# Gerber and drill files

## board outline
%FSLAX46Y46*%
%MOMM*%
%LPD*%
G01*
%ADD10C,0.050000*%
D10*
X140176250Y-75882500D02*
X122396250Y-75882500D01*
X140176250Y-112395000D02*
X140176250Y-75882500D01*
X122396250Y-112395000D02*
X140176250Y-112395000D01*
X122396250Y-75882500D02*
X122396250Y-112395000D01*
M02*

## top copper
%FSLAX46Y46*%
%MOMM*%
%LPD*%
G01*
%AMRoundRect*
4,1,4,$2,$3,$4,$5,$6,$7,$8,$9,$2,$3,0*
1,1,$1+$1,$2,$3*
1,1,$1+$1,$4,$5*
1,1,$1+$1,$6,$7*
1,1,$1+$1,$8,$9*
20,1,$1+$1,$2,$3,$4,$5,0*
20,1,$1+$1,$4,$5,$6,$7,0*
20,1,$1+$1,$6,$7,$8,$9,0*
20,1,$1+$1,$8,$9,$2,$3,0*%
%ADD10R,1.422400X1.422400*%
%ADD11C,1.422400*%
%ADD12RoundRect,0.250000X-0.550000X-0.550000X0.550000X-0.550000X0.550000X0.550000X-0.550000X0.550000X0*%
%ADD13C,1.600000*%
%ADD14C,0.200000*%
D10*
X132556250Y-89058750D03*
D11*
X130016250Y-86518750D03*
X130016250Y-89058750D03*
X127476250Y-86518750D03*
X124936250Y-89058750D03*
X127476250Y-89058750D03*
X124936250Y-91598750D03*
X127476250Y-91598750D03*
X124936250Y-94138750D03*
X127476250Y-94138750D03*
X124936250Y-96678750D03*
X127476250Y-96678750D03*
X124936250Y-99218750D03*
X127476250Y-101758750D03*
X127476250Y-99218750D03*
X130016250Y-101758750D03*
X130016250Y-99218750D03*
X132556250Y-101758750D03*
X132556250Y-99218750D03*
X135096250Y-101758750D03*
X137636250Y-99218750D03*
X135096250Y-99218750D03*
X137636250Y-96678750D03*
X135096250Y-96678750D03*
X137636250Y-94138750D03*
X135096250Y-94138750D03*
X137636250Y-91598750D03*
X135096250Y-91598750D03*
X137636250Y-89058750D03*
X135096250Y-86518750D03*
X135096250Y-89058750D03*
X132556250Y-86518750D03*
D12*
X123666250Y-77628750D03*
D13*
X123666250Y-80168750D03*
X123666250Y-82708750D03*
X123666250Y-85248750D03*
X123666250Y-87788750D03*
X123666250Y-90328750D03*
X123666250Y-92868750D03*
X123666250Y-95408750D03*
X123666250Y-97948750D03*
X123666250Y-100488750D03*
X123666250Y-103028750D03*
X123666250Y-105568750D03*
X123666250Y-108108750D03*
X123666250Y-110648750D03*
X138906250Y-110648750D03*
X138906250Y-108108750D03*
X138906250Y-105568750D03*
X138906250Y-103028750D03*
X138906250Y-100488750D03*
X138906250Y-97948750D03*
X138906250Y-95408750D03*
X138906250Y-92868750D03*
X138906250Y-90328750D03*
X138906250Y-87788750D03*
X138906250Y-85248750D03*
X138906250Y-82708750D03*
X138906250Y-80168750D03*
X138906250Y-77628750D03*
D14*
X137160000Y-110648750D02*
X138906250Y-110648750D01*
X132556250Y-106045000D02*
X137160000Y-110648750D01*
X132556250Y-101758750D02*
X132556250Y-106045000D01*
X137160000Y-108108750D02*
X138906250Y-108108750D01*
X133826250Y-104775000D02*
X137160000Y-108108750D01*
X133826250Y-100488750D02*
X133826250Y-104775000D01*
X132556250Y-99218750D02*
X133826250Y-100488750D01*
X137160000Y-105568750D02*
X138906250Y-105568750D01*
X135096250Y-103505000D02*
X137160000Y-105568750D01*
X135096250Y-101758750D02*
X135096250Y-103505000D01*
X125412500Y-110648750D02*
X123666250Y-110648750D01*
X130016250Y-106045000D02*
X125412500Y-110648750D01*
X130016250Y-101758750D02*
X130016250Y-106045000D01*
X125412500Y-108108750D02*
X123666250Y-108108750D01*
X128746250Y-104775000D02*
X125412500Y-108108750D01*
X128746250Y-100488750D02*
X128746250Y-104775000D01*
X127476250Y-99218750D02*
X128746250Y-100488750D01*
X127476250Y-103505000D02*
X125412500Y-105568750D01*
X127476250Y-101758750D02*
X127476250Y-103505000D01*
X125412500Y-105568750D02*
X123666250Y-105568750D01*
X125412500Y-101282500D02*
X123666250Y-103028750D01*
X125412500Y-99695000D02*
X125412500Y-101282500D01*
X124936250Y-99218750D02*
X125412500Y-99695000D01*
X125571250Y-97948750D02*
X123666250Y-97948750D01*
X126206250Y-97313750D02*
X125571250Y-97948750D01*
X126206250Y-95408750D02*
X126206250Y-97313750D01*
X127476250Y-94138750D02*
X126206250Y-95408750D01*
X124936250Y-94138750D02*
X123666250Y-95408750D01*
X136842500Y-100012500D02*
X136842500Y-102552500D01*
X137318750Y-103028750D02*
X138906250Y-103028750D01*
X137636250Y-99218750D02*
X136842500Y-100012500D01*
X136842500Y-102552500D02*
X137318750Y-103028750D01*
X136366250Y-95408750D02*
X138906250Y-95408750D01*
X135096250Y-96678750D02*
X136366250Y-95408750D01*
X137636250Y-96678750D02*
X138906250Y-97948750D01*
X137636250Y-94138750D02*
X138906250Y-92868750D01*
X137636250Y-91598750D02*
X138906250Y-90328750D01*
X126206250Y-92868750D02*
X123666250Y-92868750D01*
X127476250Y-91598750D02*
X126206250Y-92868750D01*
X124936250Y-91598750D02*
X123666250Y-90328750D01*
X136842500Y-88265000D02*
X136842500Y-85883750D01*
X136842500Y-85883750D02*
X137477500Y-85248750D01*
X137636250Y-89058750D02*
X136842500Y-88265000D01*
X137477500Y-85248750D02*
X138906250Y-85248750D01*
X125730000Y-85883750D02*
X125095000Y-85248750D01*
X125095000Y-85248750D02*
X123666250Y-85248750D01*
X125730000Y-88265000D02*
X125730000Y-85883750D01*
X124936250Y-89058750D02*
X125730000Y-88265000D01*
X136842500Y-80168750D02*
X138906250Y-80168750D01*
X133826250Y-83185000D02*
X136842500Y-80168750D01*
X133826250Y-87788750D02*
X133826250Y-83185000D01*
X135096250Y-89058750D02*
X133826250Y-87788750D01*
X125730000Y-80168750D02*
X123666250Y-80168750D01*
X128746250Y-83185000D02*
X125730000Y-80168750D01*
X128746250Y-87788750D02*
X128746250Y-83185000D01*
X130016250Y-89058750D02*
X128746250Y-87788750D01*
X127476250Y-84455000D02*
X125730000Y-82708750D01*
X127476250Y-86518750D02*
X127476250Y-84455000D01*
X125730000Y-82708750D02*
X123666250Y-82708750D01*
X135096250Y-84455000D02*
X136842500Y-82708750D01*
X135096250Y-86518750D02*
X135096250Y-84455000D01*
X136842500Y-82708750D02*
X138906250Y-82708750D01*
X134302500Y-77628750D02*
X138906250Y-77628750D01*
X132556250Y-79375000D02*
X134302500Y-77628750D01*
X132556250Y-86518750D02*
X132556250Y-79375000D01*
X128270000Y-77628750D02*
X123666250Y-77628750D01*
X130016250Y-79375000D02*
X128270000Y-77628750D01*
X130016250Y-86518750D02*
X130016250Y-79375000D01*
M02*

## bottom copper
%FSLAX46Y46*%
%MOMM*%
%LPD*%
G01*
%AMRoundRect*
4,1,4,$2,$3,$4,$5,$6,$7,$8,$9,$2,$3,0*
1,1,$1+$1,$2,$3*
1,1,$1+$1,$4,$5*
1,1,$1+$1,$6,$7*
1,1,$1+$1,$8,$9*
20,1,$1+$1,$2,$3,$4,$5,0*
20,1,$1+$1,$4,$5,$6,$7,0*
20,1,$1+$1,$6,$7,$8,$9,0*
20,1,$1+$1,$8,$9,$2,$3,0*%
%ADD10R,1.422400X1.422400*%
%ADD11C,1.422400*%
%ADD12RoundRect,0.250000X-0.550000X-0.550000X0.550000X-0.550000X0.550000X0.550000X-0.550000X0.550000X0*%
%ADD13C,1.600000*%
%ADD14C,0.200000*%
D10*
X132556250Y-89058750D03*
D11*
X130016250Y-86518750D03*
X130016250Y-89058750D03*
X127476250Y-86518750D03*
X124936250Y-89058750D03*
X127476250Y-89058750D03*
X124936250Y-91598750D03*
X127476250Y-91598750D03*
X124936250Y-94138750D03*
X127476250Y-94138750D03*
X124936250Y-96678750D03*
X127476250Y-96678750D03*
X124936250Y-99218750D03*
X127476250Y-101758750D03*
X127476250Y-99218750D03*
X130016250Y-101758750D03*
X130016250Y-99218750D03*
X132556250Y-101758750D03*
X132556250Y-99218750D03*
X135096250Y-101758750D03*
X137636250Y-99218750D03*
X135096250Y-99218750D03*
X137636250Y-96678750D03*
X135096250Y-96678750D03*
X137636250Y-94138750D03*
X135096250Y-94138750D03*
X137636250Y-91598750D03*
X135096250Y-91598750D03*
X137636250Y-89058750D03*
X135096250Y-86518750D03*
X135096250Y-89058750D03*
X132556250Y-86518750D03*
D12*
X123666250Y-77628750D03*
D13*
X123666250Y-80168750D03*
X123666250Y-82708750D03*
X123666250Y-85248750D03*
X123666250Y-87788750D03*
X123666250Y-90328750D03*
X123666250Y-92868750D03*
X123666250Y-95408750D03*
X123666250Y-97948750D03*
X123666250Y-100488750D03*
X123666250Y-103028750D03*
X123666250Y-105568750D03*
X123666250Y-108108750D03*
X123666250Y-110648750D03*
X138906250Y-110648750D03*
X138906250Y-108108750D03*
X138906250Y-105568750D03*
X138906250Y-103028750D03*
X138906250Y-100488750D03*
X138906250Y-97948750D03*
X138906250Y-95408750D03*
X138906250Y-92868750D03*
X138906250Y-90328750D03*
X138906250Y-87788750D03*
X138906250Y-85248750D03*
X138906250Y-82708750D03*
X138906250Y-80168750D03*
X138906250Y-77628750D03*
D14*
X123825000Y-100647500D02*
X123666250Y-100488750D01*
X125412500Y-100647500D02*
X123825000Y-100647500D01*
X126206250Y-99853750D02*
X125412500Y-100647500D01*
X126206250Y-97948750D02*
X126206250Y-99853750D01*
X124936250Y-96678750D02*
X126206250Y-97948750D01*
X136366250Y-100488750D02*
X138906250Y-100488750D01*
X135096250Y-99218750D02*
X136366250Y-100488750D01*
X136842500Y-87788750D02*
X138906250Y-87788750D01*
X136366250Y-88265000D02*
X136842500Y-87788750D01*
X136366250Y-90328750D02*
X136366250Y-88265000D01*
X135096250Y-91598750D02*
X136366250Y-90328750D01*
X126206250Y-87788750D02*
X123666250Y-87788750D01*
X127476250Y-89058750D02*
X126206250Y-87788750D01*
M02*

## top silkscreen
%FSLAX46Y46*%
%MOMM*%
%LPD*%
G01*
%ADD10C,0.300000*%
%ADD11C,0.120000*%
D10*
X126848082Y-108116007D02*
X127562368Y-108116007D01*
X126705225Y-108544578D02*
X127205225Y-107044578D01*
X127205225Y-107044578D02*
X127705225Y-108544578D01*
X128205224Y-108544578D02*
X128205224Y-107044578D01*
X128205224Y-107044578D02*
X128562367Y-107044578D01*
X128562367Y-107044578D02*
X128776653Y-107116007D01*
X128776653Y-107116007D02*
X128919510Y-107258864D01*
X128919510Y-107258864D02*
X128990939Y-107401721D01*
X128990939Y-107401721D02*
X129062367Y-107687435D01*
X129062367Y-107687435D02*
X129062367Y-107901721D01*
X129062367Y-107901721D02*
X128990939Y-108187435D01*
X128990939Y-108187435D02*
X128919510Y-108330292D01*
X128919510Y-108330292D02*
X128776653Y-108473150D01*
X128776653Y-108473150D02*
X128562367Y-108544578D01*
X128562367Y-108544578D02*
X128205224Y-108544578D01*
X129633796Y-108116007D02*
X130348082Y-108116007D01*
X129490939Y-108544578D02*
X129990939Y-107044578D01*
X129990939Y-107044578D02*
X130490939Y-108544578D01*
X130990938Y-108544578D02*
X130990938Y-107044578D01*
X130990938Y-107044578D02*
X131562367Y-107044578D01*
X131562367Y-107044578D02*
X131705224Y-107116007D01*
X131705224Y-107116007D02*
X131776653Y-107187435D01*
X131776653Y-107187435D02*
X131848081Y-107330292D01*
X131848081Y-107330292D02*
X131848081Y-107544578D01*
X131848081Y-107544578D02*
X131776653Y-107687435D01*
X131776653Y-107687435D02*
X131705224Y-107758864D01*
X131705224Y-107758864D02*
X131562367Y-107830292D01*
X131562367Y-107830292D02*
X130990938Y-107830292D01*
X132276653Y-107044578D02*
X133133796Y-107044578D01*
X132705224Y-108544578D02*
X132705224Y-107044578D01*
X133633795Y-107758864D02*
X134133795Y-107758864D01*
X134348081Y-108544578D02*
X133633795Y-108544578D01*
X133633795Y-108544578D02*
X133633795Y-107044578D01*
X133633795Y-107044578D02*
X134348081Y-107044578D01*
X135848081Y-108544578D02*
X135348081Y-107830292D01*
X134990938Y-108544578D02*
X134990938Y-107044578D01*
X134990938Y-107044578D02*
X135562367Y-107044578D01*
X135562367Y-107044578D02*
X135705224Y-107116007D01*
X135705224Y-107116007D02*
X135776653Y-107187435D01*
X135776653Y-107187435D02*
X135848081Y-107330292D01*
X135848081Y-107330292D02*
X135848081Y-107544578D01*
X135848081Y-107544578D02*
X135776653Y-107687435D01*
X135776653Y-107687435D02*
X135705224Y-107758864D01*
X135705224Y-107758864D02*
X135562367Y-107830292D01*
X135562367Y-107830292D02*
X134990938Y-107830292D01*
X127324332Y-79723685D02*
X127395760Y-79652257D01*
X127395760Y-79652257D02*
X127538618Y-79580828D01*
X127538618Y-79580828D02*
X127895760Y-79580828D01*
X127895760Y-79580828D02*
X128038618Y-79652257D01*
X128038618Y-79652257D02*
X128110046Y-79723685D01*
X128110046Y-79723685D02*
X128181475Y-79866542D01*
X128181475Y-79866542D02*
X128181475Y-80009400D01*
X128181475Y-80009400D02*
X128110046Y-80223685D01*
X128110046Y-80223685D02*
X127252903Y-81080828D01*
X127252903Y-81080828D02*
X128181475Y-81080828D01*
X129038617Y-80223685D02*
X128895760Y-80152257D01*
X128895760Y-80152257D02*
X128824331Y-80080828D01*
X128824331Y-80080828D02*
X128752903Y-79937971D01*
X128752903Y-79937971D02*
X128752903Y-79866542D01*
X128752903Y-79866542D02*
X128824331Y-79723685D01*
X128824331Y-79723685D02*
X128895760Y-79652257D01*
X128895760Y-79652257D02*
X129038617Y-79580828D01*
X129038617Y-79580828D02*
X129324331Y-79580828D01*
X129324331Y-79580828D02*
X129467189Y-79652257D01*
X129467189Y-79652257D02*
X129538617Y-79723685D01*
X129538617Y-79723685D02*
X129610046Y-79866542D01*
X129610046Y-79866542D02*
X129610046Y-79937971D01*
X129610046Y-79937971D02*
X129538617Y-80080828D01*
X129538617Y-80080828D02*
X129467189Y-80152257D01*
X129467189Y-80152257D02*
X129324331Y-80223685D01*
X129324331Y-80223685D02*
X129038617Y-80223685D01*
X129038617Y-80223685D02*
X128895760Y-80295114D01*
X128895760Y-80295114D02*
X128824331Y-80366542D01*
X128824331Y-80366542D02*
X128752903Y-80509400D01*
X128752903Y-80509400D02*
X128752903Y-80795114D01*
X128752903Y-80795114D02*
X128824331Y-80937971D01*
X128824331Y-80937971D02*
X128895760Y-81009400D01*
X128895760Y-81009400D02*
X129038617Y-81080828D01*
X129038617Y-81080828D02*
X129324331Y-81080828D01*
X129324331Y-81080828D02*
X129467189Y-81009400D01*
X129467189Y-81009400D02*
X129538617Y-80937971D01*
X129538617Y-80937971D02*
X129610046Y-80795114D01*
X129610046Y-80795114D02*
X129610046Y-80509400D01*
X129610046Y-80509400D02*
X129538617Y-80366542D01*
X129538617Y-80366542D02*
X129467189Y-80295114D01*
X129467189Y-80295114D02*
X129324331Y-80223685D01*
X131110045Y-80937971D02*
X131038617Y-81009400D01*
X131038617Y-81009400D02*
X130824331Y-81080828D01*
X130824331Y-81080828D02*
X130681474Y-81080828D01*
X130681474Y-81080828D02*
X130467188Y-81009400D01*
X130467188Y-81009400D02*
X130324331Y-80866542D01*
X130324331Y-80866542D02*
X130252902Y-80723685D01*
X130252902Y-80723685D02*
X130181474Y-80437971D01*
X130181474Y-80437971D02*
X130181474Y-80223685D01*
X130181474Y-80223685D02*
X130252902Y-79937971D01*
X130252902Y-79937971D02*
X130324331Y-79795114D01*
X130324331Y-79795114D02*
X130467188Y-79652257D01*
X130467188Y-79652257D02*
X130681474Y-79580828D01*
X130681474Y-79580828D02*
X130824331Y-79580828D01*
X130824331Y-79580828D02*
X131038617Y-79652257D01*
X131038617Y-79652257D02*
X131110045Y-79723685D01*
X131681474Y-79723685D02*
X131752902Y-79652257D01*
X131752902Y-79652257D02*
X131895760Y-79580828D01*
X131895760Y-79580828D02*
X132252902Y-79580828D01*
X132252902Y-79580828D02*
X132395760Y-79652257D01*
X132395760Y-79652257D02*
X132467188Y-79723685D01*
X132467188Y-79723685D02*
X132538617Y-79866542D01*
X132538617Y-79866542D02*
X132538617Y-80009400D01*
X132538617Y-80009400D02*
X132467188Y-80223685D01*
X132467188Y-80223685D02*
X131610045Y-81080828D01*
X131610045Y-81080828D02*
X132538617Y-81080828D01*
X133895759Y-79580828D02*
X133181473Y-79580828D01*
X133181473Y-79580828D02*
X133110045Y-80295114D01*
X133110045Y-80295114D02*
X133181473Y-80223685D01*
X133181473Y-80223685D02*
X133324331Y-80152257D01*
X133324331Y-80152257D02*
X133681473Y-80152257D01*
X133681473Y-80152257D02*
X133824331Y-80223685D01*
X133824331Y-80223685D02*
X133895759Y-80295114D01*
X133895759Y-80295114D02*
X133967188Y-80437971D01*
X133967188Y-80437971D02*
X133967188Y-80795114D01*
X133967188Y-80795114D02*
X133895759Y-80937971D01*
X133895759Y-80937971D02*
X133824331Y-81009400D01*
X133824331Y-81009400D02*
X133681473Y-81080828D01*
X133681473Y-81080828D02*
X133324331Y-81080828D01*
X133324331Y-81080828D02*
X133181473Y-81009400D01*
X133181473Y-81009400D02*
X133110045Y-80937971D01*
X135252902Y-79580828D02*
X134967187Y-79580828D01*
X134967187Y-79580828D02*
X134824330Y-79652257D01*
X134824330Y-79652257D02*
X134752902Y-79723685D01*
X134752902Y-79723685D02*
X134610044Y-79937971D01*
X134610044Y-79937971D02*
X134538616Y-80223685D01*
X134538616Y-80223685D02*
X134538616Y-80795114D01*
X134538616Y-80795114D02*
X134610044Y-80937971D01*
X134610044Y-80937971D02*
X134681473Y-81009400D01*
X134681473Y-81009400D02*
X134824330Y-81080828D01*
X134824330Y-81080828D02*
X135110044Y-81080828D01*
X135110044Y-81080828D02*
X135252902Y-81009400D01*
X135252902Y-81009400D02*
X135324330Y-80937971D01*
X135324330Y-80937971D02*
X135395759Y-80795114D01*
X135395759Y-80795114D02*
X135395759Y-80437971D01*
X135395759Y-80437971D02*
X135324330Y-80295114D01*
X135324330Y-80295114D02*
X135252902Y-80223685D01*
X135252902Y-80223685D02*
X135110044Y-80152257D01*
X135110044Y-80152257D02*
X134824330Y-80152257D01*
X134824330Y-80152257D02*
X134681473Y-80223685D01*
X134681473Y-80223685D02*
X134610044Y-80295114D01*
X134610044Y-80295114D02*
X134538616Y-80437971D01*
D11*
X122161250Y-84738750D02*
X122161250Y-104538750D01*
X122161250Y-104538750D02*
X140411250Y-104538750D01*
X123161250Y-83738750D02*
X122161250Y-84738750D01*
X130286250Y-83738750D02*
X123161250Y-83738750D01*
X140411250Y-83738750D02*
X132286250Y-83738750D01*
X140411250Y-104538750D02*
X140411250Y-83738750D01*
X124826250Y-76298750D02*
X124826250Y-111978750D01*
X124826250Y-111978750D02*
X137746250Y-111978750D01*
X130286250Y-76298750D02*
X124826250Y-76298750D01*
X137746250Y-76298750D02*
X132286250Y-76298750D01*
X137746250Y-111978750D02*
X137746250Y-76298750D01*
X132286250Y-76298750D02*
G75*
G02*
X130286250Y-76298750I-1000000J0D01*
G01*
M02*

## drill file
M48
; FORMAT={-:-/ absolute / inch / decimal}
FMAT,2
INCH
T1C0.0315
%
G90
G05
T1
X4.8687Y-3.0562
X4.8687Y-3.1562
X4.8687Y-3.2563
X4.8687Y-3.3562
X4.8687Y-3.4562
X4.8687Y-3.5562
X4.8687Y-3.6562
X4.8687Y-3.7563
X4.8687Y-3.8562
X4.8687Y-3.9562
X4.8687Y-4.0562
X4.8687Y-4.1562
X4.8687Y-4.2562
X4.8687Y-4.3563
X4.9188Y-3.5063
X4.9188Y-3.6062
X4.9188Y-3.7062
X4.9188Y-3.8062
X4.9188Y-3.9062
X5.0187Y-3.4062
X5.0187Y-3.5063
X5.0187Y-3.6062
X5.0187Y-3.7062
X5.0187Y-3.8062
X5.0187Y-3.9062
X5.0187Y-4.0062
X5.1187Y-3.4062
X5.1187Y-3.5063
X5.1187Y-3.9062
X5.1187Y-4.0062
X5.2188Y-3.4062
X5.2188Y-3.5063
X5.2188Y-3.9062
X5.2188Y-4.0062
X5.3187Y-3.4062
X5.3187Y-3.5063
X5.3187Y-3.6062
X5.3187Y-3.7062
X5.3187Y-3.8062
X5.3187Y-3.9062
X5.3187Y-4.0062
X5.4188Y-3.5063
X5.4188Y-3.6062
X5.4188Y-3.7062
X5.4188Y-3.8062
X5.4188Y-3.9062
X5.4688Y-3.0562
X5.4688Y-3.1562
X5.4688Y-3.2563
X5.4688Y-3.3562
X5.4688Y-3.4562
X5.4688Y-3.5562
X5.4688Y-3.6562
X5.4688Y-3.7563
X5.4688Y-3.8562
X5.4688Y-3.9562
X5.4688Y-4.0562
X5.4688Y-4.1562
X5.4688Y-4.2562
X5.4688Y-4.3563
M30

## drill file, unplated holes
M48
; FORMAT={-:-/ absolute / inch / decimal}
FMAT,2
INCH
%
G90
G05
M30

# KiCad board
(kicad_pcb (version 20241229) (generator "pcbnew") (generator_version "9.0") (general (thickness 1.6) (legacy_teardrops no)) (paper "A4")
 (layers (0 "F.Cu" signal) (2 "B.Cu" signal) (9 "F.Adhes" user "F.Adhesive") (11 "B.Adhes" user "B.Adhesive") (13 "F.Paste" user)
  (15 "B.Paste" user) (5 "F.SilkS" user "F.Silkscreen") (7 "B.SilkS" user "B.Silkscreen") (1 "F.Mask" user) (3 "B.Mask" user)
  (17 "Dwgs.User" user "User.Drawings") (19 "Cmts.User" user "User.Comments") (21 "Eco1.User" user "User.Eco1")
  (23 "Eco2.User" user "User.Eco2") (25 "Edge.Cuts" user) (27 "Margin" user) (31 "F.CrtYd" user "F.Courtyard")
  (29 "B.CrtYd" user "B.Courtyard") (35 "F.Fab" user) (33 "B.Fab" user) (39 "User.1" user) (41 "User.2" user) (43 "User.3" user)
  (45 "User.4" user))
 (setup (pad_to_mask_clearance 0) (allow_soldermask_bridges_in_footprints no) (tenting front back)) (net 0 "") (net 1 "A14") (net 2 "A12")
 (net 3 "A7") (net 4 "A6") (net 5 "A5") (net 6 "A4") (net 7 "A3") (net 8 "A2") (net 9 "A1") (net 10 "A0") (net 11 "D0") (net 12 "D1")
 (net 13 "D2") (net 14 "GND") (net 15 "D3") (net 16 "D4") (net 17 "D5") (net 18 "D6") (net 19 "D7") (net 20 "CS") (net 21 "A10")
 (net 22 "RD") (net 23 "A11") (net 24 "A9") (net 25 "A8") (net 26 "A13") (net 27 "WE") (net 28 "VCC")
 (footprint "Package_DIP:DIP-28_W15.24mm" (layer "F.Cu") (at 123.66625 77.62875)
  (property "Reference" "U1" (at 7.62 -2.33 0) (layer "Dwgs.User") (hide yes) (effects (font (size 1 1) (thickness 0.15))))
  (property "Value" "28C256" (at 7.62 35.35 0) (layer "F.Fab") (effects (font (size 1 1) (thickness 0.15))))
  (fp_line (start 1.16 -1.33) (end 1.16 34.35) (stroke (width 0.12) (type solid)) (layer "F.SilkS"))
  (fp_line (start 1.16 34.35) (end 14.08 34.35) (stroke (width 0.12) (type solid)) (layer "F.SilkS"))
  (fp_line (start 6.62 -1.33) (end 1.16 -1.33) (stroke (width 0.12) (type solid)) (layer "F.SilkS"))
  (fp_line (start 14.08 -1.33) (end 8.62 -1.33) (stroke (width 0.12) (type solid)) (layer "F.SilkS"))
  (fp_line (start 14.08 34.35) (end 14.08 -1.33) (stroke (width 0.12) (type solid)) (layer "F.SilkS"))
  (fp_arc (start 8.62 -1.33) (mid 7.62 -0.33) (end 6.62 -1.33) (stroke (width 0.12) (type solid)) (layer "F.SilkS"))
  (pad "1" thru_hole roundrect (at 0 0) (size 1.6 1.6) (drill 0.8) (layers "*.Cu" "*.Mask") (remove_unused_layers no)
   (roundrect_rratio 0.15625) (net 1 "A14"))
  (pad "2" thru_hole circle (at 0 2.54) (size 1.6 1.6) (drill 0.8) (layers "*.Cu" "*.Mask") (remove_unused_layers no) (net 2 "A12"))
  (pad "3" thru_hole circle (at 0 5.08) (size 1.6 1.6) (drill 0.8) (layers "*.Cu" "*.Mask") (remove_unused_layers no) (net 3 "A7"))
  (pad "4" thru_hole circle (at 0 7.62) (size 1.6 1.6) (drill 0.8) (layers "*.Cu" "*.Mask") (remove_unused_layers no) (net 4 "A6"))
  (pad "5" thru_hole circle (at 0 10.16) (size 1.6 1.6) (drill 0.8) (layers "*.Cu" "*.Mask") (remove_unused_layers no) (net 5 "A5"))
  (pad "6" thru_hole circle (at 0 12.7) (size 1.6 1.6) (drill 0.8) (layers "*.Cu" "*.Mask") (remove_unused_layers no) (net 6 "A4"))
  (pad "7" thru_hole circle (at 0 15.24) (size 1.6 1.6) (drill 0.8) (layers "*.Cu" "*.Mask") (remove_unused_layers no) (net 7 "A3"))
  (pad "8" thru_hole circle (at 0 17.78) (size 1.6 1.6) (drill 0.8) (layers "*.Cu" "*.Mask") (remove_unused_layers no) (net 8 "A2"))
  (pad "9" thru_hole circle (at 0 20.32) (size 1.6 1.6) (drill 0.8) (layers "*.Cu" "*.Mask") (remove_unused_layers no) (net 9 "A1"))
  (pad "10" thru_hole circle (at 0 22.86) (size 1.6 1.6) (drill 0.8) (layers "*.Cu" "*.Mask") (remove_unused_layers no) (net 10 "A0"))
  (pad "11" thru_hole circle (at 0 25.4) (size 1.6 1.6) (drill 0.8) (layers "*.Cu" "*.Mask") (remove_unused_layers no) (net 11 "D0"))
  (pad "12" thru_hole circle (at 0 27.94) (size 1.6 1.6) (drill 0.8) (layers "*.Cu" "*.Mask") (remove_unused_layers no) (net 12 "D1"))
  (pad "13" thru_hole circle (at 0 30.48) (size 1.6 1.6) (drill 0.8) (layers "*.Cu" "*.Mask") (remove_unused_layers no) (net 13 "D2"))
  (pad "14" thru_hole circle (at 0 33.02) (size 1.6 1.6) (drill 0.8) (layers "*.Cu" "*.Mask") (remove_unused_layers no) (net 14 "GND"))
  (pad "15" thru_hole circle (at 15.24 33.02) (size 1.6 1.6) (drill 0.8) (layers "*.Cu" "*.Mask") (remove_unused_layers no) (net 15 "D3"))
  (pad "16" thru_hole circle (at 15.24 30.48) (size 1.6 1.6) (drill 0.8) (layers "*.Cu" "*.Mask") (remove_unused_layers no) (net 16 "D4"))
  (pad "17" thru_hole circle (at 15.24 27.94) (size 1.6 1.6) (drill 0.8) (layers "*.Cu" "*.Mask") (remove_unused_layers no) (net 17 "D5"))
  (pad "18" thru_hole circle (at 15.24 25.4) (size 1.6 1.6) (drill 0.8) (layers "*.Cu" "*.Mask") (remove_unused_layers no) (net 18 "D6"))
  (pad "19" thru_hole circle (at 15.24 22.86) (size 1.6 1.6) (drill 0.8) (layers "*.Cu" "*.Mask") (remove_unused_layers no) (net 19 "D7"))
  (pad "20" thru_hole circle (at 15.24 20.32) (size 1.6 1.6) (drill 0.8) (layers "*.Cu" "*.Mask") (remove_unused_layers no) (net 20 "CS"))
  (pad "21" thru_hole circle (at 15.24 17.78) (size 1.6 1.6) (drill 0.8) (layers "*.Cu" "*.Mask") (remove_unused_layers no) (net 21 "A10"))
  (pad "22" thru_hole circle (at 15.24 15.24) (size 1.6 1.6) (drill 0.8) (layers "*.Cu" "*.Mask") (remove_unused_layers no) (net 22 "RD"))
  (pad "23" thru_hole circle (at 15.24 12.7) (size 1.6 1.6) (drill 0.8) (layers "*.Cu" "*.Mask") (remove_unused_layers no) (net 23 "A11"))
  (pad "24" thru_hole circle (at 15.24 10.16) (size 1.6 1.6) (drill 0.8) (layers "*.Cu" "*.Mask") (remove_unused_layers no) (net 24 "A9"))
  (pad "25" thru_hole circle (at 15.24 7.62) (size 1.6 1.6) (drill 0.8) (layers "*.Cu" "*.Mask") (remove_unused_layers no) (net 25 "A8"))
  (pad "26" thru_hole circle (at 15.24 5.08) (size 1.6 1.6) (drill 0.8) (layers "*.Cu" "*.Mask") (remove_unused_layers no) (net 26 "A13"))
  (pad "27" thru_hole circle (at 15.24 2.54) (size 1.6 1.6) (drill 0.8) (layers "*.Cu" "*.Mask") (remove_unused_layers no) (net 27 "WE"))
  (pad "28" thru_hole circle (at 15.24 0) (size 1.6 1.6) (drill 0.8) (layers "*.Cu" "*.Mask") (remove_unused_layers no) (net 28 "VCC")))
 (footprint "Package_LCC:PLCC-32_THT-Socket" (layer "F.Cu") (at 132.55625 89.05875)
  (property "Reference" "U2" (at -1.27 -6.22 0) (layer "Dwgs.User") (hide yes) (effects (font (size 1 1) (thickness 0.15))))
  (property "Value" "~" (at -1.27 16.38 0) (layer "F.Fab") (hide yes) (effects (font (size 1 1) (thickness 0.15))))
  (fp_line (start -10.395 -4.32) (end -10.395 15.48) (stroke (width 0.12) (type solid)) (layer "F.SilkS"))
  (fp_line (start -10.395 15.48) (end 7.855 15.48) (stroke (width 0.12) (type solid)) (layer "F.SilkS"))
  (fp_line (start -9.395 -5.32) (end -10.395 -4.32) (stroke (width 0.12) (type solid)) (layer "F.SilkS"))
  (fp_line (start -2.27 -5.32) (end -9.395 -5.32) (stroke (width 0.12) (type solid)) (layer "F.SilkS"))
  (fp_line (start 7.855 -5.32) (end -0.27 -5.32) (stroke (width 0.12) (type solid)) (layer "F.SilkS"))
  (fp_line (start 7.855 15.48) (end 7.855 -5.32) (stroke (width 0.12) (type solid)) (layer "F.SilkS"))
  (pad "1" thru_hole rect (at 0 0) (size 1.4224 1.4224) (drill 0.8) (layers "*.Cu" "*.Mask") (remove_unused_layers no))
  (pad "2" thru_hole circle (at -2.54 -2.54) (size 1.4224 1.4224) (drill 0.8) (layers "*.Cu" "*.Mask") (remove_unused_layers no)
   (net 1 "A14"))
  (pad "3" thru_hole circle (at -2.54 0) (size 1.4224 1.4224) (drill 0.8) (layers "*.Cu" "*.Mask") (remove_unused_layers no) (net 2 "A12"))
  (pad "4" thru_hole circle (at -5.08 -2.54) (size 1.4224 1.4224) (drill 0.8) (layers "*.Cu" "*.Mask") (remove_unused_layers no)
   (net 3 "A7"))
  (pad "5" thru_hole circle (at -7.62 0) (size 1.4224 1.4224) (drill 0.8) (layers "*.Cu" "*.Mask") (remove_unused_layers no) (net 4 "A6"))
  (pad "6" thru_hole circle (at -5.08 0) (size 1.4224 1.4224) (drill 0.8) (layers "*.Cu" "*.Mask") (remove_unused_layers no) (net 5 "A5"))
  (pad "7" thru_hole circle (at -7.62 2.54) (size 1.4224 1.4224) (drill 0.8) (layers "*.Cu" "*.Mask") (remove_unused_layers no) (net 6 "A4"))
  (pad "8" thru_hole circle (at -5.08 2.54) (size 1.4224 1.4224) (drill 0.8) (layers "*.Cu" "*.Mask") (remove_unused_layers no) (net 7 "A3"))
  (pad "9" thru_hole circle (at -7.62 5.08) (size 1.4224 1.4224) (drill 0.8) (layers "*.Cu" "*.Mask") (remove_unused_layers no) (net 8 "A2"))
  (pad "10" thru_hole circle (at -5.08 5.08) (size 1.4224 1.4224) (drill 0.8) (layers "*.Cu" "*.Mask") (remove_unused_layers no)
   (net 9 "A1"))
  (pad "11" thru_hole circle (at -7.62 7.62) (size 1.4224 1.4224) (drill 0.8) (layers "*.Cu" "*.Mask") (remove_unused_layers no)
   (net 10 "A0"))
  (pad "12" thru_hole circle (at -5.08 7.62) (size 1.4224 1.4224) (drill 0.8) (layers "*.Cu" "*.Mask") (remove_unused_layers no))
  (pad "13" thru_hole circle (at -7.62 10.16) (size 1.4224 1.4224) (drill 0.8) (layers "*.Cu" "*.Mask") (remove_unused_layers no)
   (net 11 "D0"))
  (pad "14" thru_hole circle (at -5.08 12.7) (size 1.4224 1.4224) (drill 0.8) (layers "*.Cu" "*.Mask") (remove_unused_layers no)
   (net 12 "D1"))
  (pad "15" thru_hole circle (at -5.08 10.16) (size 1.4224 1.4224) (drill 0.8) (layers "*.Cu" "*.Mask") (remove_unused_layers no)
   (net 13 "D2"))
  (pad "16" thru_hole circle (at -2.54 12.7) (size 1.4224 1.4224) (drill 0.8) (layers "*.Cu" "*.Mask") (remove_unused_layers no)
   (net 14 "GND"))
  (pad "17" thru_hole circle (at -2.54 10.16) (size 1.4224 1.4224) (drill 0.8) (layers "*.Cu" "*.Mask") (remove_unused_layers no))
  (pad "18" thru_hole circle (at 0 12.7) (size 1.4224 1.4224) (drill 0.8) (layers "*.Cu" "*.Mask") (remove_unused_layers no) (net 15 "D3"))
  (pad "19" thru_hole circle (at 0 10.16) (size 1.4224 1.4224) (drill 0.8) (layers "*.Cu" "*.Mask") (remove_unused_layers no) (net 16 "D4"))
  (pad "20" thru_hole circle (at 2.54 12.7) (size 1.4224 1.4224) (drill 0.8) (layers "*.Cu" "*.Mask") (remove_unused_layers no)
   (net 17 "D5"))
  (pad "21" thru_hole circle (at 5.08 10.16) (size 1.4224 1.4224) (drill 0.8) (layers "*.Cu" "*.Mask") (remove_unused_layers no)
   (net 18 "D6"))
  (pad "22" thru_hole circle (at 2.54 10.16) (size 1.4224 1.4224) (drill 0.8) (layers "*.Cu" "*.Mask") (remove_unused_layers no)
   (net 19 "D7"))
  (pad "23" thru_hole circle (at 5.08 7.62) (size 1.4224 1.4224) (drill 0.8) (layers "*.Cu" "*.Mask") (remove_unused_layers no)
   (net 20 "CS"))
  (pad "24" thru_hole circle (at 2.54 7.62) (size 1.4224 1.4224) (drill 0.8) (layers "*.Cu" "*.Mask") (remove_unused_layers no)
   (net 21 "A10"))
  (pad "25" thru_hole circle (at 5.08 5.08) (size 1.4224 1.4224) (drill 0.8) (layers "*.Cu" "*.Mask") (remove_unused_layers no)
   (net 22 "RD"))
  (pad "26" thru_hole circle (at 2.54 5.08) (size 1.4224 1.4224) (drill 0.8) (layers "*.Cu" "*.Mask") (remove_unused_layers no))
  (pad "27" thru_hole circle (at 5.08 2.54) (size 1.4224 1.4224) (drill 0.8) (layers "*.Cu" "*.Mask") (remove_unused_layers no)
   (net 23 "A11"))
  (pad "28" thru_hole circle (at 2.54 2.54) (size 1.4224 1.4224) (drill 0.8) (layers "*.Cu" "*.Mask") (remove_unused_layers no)
   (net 24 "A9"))
  (pad "29" thru_hole circle (at 5.08 0) (size 1.4224 1.4224) (drill 0.8) (layers "*.Cu" "*.Mask") (remove_unused_layers no) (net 25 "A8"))
  (pad "30" thru_hole circle (at 2.54 -2.54) (size 1.4224 1.4224) (drill 0.8) (layers "*.Cu" "*.Mask") (remove_unused_layers no)
   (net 26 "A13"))
  (pad "31" thru_hole circle (at 2.54 0) (size 1.4224 1.4224) (drill 0.8) (layers "*.Cu" "*.Mask") (remove_unused_layers no) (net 27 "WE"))
  (pad "32" thru_hole circle (at 0 -2.54) (size 1.4224 1.4224) (drill 0.8) (layers "*.Cu" "*.Mask") (remove_unused_layers no) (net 28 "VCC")))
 (gr_line (start 122.39625 112.395) (end 140.17625 112.395) (stroke (width 0.05) (type default)) (layer "Edge.Cuts"))
 (gr_line (start 140.17625 75.8825) (end 122.39625 75.8825) (stroke (width 0.05) (type default)) (layer "Edge.Cuts"))
 (gr_line (start 122.39625 75.8825) (end 122.39625 112.395) (stroke (width 0.05) (type default)) (layer "Edge.Cuts"))
 (gr_line (start 140.17625 112.395) (end 140.17625 75.8825) (stroke (width 0.05) (type default)) (layer "Edge.Cuts"))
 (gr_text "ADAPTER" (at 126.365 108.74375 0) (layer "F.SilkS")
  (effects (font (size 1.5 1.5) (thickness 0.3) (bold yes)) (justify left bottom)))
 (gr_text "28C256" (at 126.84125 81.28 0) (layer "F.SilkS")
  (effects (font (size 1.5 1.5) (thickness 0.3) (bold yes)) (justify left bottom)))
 (segment (start 130.01625 106.045) (end 125.4125 110.64875) (width 0.2) (layer "F.Cu") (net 14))
 (segment (start 125.4125 110.64875) (end 123.66625 110.64875) (width 0.2) (layer "F.Cu") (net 14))
 (segment (start 130.01625 101.75875) (end 130.01625 106.045) (width 0.2) (layer "F.Cu") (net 14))
 (segment (start 125.57125 97.94875) (end 123.66625 97.94875) (width 0.2) (layer "F.Cu") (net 9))
 (segment (start 126.20625 95.40875) (end 126.20625 97.31375) (width 0.2) (layer "F.Cu") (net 9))
 (segment (start 127.47625 94.13875) (end 126.20625 95.40875) (width 0.2) (layer "F.Cu") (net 9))
 (segment (start 126.20625 97.31375) (end 125.57125 97.94875) (width 0.2) (layer "F.Cu") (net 9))
 (segment (start 124.93625 91.59875) (end 123.66625 90.32875) (width 0.2) (layer "F.Cu") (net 6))
 (segment (start 125.4125 101.2825) (end 123.66625 103.02875) (width 0.2) (layer "F.Cu") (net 11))
 (segment (start 125.4125 99.695) (end 125.4125 101.2825) (width 0.2) (layer "F.Cu") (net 11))
 (segment (start 124.93625 99.21875) (end 125.4125 99.695) (width 0.2) (layer "F.Cu") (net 11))
 (segment (start 135.09625 91.59875) (end 136.36625 90.32875) (width 0.2) (layer "B.Cu") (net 24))
 (segment (start 136.36625 88.265) (end 136.8425 87.78875) (width 0.2) (layer "B.Cu") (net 24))
 (segment (start 136.36625 90.32875) (end 136.36625 88.265) (width 0.2) (layer "B.Cu") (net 24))
 (segment (start 136.8425 87.78875) (end 138.90625 87.78875) (width 0.2) (layer "B.Cu") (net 24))
 (segment (start 137.63625 96.67875) (end 138.90625 97.94875) (width 0.2) (layer "F.Cu") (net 20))
 (segment (start 128.74625 87.78875) (end 128.74625 83.185) (width 0.2) (layer "F.Cu") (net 2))
 (segment (start 125.73 80.16875) (end 123.66625 80.16875) (width 0.2) (layer "F.Cu") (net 2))
 (segment (start 130.01625 89.05875) (end 128.74625 87.78875) (width 0.2) (layer "F.Cu") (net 2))
 (segment (start 128.74625 83.185) (end 125.73 80.16875) (width 0.2) (layer "F.Cu") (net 2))
 (segment (start 136.8425 85.88375) (end 137.4775 85.24875) (width 0.2) (layer "F.Cu") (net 25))
 (segment (start 137.63625 89.05875) (end 136.8425 88.265) (width 0.2) (layer "F.Cu") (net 25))
 (segment (start 136.8425 88.265) (end 136.8425 85.88375) (width 0.2) (layer "F.Cu") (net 25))
 (segment (start 137.4775 85.24875) (end 138.90625 85.24875) (width 0.2) (layer "F.Cu") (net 25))
 (segment (start 133.82625 83.185) (end 136.8425 80.16875) (width 0.2) (layer "F.Cu") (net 27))
 (segment (start 133.82625 87.78875) (end 133.82625 83.185) (width 0.2) (layer "F.Cu") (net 27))
 (segment (start 135.09625 89.05875) (end 133.82625 87.78875) (width 0.2) (layer "F.Cu") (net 27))
 (segment (start 136.8425 80.16875) (end 138.90625 80.16875) (width 0.2) (layer "F.Cu") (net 27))
 (segment (start 134.3025 77.62875) (end 138.90625 77.62875) (width 0.2) (layer "F.Cu") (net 28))
 (segment (start 132.55625 86.51875) (end 132.55625 79.375) (width 0.2) (layer "F.Cu") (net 28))
 (segment (start 132.55625 79.375) (end 134.3025 77.62875) (width 0.2) (layer "F.Cu") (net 28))
 (segment (start 125.73 82.70875) (end 123.66625 82.70875) (width 0.2) (layer "F.Cu") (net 3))
 (segment (start 127.47625 86.51875) (end 127.47625 84.455) (width 0.2) (layer "F.Cu") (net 3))
 (segment (start 127.47625 84.455) (end 125.73 82.70875) (width 0.2) (layer "F.Cu") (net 3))
 (segment (start 136.36625 100.48875) (end 138.90625 100.48875) (width 0.2) (layer "B.Cu") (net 19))
 (segment (start 135.09625 99.21875) (end 136.36625 100.48875) (width 0.2) (layer "B.Cu") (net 19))
 (segment (start 130.01625 79.375) (end 128.27 77.62875) (width 0.2) (layer "F.Cu") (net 1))
 (segment (start 130.01625 86.51875) (end 130.01625 79.375) (width 0.2) (layer "F.Cu") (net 1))
 (segment (start 128.27 77.62875) (end 123.66625 77.62875) (width 0.2) (layer "F.Cu") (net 1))
 (segment (start 127.47625 101.75875) (end 127.47625 103.505) (width 0.2) (layer "F.Cu") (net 12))
 (segment (start 125.4125 105.56875) (end 123.66625 105.56875) (width 0.2) (layer "F.Cu") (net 12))
 (segment (start 127.47625 103.505) (end 125.4125 105.56875) (width 0.2) (layer "F.Cu") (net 12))
 (segment (start 126.20625 92.86875) (end 123.66625 92.86875) (width 0.2) (layer "F.Cu") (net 7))
 (segment (start 127.47625 91.59875) (end 126.20625 92.86875) (width 0.2) (layer "F.Cu") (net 7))
 (segment (start 124.93625 89.05875) (end 125.73 88.265) (width 0.2) (layer "F.Cu") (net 4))
 (segment (start 125.095 85.24875) (end 123.66625 85.24875) (width 0.2) (layer "F.Cu") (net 4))
 (segment (start 125.73 85.88375) (end 125.095 85.24875) (width 0.2) (layer "F.Cu") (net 4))
 (segment (start 125.73 88.265) (end 125.73 85.88375) (width 0.2) (layer "F.Cu") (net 4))
 (segment (start 136.8425 102.5525) (end 137.31875 103.02875) (width 0.2) (layer "F.Cu") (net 18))
 (segment (start 137.31875 103.02875) (end 138.90625 103.02875) (width 0.2) (layer "F.Cu") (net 18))
 (segment (start 136.8425 100.0125) (end 136.8425 102.5525) (width 0.2) (layer "F.Cu") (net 18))
 (segment (start 137.63625 99.21875) (end 136.8425 100.0125) (width 0.2) (layer "F.Cu") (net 18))
 (segment (start 127.47625 89.05875) (end 126.20625 87.78875) (width 0.2) (layer "B.Cu") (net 5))
 (segment (start 126.20625 87.78875) (end 123.66625 87.78875) (width 0.2) (layer "B.Cu") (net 5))
 (segment (start 135.09625 84.455) (end 136.8425 82.70875) (width 0.2) (layer "F.Cu") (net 26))
 (segment (start 136.8425 82.70875) (end 138.90625 82.70875) (width 0.2) (layer "F.Cu") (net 26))
 (segment (start 135.09625 86.51875) (end 135.09625 84.455) (width 0.2) (layer "F.Cu") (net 26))
 (segment (start 133.82625 100.48875) (end 133.82625 104.775) (width 0.2) (layer "F.Cu") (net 16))
 (segment (start 132.55625 99.21875) (end 133.82625 100.48875) (width 0.2) (layer "F.Cu") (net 16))
 (segment (start 137.16 108.10875) (end 138.90625 108.10875) (width 0.2) (layer "F.Cu") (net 16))
 (segment (start 133.82625 104.775) (end 137.16 108.10875) (width 0.2) (layer "F.Cu") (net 16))
 (segment (start 132.55625 101.75875) (end 132.55625 106.045) (width 0.2) (layer "F.Cu") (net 15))
 (segment (start 137.16 110.64875) (end 138.90625 110.64875) (width 0.2) (layer "F.Cu") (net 15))
 (segment (start 132.55625 106.045) (end 137.16 110.64875) (width 0.2) (layer "F.Cu") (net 15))
 (segment (start 137.16 105.56875) (end 138.90625 105.56875) (width 0.2) (layer "F.Cu") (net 17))
 (segment (start 135.09625 101.75875) (end 135.09625 103.505) (width 0.2) (layer "F.Cu") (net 17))
 (segment (start 135.09625 103.505) (end 137.16 105.56875) (width 0.2) (layer "F.Cu") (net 17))
 (segment (start 137.63625 94.13875) (end 138.90625 92.86875) (width 0.2) (layer "F.Cu") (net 22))
 (segment (start 128.74625 104.775) (end 125.4125 108.10875) (width 0.2) (layer "F.Cu") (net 13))
 (segment (start 127.47625 99.21875) (end 128.74625 100.48875) (width 0.2) (layer "F.Cu") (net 13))
 (segment (start 128.74625 100.48875) (end 128.74625 104.775) (width 0.2) (layer "F.Cu") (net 13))
 (segment (start 125.4125 108.10875) (end 123.66625 108.10875) (width 0.2) (layer "F.Cu") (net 13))
 (segment (start 124.93625 94.13875) (end 123.66625 95.40875) (width 0.2) (layer "F.Cu") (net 8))
 (segment (start 137.63625 91.59875) (end 138.90625 90.32875) (width 0.2) (layer "F.Cu") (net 23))
 (segment (start 136.36625 95.40875) (end 138.90625 95.40875) (width 0.2) (layer "F.Cu") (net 21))
 (segment (start 135.09625 96.67875) (end 136.36625 95.40875) (width 0.2) (layer "F.Cu") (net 21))
 (segment (start 126.20625 99.85375) (end 125.4125 100.6475) (width 0.2) (layer "B.Cu") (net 10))
 (segment (start 125.4125 100.6475) (end 123.825 100.6475) (width 0.2) (layer "B.Cu") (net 10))
 (segment (start 124.93625 96.67875) (end 126.20625 97.94875) (width 0.2) (layer "B.Cu") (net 10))
 (segment (start 126.20625 97.94875) (end 126.20625 99.85375) (width 0.2) (layer "B.Cu") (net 10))
 (segment (start 123.825 100.6475) (end 123.66625 100.48875) (width 0.2) (layer "B.Cu") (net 10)))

